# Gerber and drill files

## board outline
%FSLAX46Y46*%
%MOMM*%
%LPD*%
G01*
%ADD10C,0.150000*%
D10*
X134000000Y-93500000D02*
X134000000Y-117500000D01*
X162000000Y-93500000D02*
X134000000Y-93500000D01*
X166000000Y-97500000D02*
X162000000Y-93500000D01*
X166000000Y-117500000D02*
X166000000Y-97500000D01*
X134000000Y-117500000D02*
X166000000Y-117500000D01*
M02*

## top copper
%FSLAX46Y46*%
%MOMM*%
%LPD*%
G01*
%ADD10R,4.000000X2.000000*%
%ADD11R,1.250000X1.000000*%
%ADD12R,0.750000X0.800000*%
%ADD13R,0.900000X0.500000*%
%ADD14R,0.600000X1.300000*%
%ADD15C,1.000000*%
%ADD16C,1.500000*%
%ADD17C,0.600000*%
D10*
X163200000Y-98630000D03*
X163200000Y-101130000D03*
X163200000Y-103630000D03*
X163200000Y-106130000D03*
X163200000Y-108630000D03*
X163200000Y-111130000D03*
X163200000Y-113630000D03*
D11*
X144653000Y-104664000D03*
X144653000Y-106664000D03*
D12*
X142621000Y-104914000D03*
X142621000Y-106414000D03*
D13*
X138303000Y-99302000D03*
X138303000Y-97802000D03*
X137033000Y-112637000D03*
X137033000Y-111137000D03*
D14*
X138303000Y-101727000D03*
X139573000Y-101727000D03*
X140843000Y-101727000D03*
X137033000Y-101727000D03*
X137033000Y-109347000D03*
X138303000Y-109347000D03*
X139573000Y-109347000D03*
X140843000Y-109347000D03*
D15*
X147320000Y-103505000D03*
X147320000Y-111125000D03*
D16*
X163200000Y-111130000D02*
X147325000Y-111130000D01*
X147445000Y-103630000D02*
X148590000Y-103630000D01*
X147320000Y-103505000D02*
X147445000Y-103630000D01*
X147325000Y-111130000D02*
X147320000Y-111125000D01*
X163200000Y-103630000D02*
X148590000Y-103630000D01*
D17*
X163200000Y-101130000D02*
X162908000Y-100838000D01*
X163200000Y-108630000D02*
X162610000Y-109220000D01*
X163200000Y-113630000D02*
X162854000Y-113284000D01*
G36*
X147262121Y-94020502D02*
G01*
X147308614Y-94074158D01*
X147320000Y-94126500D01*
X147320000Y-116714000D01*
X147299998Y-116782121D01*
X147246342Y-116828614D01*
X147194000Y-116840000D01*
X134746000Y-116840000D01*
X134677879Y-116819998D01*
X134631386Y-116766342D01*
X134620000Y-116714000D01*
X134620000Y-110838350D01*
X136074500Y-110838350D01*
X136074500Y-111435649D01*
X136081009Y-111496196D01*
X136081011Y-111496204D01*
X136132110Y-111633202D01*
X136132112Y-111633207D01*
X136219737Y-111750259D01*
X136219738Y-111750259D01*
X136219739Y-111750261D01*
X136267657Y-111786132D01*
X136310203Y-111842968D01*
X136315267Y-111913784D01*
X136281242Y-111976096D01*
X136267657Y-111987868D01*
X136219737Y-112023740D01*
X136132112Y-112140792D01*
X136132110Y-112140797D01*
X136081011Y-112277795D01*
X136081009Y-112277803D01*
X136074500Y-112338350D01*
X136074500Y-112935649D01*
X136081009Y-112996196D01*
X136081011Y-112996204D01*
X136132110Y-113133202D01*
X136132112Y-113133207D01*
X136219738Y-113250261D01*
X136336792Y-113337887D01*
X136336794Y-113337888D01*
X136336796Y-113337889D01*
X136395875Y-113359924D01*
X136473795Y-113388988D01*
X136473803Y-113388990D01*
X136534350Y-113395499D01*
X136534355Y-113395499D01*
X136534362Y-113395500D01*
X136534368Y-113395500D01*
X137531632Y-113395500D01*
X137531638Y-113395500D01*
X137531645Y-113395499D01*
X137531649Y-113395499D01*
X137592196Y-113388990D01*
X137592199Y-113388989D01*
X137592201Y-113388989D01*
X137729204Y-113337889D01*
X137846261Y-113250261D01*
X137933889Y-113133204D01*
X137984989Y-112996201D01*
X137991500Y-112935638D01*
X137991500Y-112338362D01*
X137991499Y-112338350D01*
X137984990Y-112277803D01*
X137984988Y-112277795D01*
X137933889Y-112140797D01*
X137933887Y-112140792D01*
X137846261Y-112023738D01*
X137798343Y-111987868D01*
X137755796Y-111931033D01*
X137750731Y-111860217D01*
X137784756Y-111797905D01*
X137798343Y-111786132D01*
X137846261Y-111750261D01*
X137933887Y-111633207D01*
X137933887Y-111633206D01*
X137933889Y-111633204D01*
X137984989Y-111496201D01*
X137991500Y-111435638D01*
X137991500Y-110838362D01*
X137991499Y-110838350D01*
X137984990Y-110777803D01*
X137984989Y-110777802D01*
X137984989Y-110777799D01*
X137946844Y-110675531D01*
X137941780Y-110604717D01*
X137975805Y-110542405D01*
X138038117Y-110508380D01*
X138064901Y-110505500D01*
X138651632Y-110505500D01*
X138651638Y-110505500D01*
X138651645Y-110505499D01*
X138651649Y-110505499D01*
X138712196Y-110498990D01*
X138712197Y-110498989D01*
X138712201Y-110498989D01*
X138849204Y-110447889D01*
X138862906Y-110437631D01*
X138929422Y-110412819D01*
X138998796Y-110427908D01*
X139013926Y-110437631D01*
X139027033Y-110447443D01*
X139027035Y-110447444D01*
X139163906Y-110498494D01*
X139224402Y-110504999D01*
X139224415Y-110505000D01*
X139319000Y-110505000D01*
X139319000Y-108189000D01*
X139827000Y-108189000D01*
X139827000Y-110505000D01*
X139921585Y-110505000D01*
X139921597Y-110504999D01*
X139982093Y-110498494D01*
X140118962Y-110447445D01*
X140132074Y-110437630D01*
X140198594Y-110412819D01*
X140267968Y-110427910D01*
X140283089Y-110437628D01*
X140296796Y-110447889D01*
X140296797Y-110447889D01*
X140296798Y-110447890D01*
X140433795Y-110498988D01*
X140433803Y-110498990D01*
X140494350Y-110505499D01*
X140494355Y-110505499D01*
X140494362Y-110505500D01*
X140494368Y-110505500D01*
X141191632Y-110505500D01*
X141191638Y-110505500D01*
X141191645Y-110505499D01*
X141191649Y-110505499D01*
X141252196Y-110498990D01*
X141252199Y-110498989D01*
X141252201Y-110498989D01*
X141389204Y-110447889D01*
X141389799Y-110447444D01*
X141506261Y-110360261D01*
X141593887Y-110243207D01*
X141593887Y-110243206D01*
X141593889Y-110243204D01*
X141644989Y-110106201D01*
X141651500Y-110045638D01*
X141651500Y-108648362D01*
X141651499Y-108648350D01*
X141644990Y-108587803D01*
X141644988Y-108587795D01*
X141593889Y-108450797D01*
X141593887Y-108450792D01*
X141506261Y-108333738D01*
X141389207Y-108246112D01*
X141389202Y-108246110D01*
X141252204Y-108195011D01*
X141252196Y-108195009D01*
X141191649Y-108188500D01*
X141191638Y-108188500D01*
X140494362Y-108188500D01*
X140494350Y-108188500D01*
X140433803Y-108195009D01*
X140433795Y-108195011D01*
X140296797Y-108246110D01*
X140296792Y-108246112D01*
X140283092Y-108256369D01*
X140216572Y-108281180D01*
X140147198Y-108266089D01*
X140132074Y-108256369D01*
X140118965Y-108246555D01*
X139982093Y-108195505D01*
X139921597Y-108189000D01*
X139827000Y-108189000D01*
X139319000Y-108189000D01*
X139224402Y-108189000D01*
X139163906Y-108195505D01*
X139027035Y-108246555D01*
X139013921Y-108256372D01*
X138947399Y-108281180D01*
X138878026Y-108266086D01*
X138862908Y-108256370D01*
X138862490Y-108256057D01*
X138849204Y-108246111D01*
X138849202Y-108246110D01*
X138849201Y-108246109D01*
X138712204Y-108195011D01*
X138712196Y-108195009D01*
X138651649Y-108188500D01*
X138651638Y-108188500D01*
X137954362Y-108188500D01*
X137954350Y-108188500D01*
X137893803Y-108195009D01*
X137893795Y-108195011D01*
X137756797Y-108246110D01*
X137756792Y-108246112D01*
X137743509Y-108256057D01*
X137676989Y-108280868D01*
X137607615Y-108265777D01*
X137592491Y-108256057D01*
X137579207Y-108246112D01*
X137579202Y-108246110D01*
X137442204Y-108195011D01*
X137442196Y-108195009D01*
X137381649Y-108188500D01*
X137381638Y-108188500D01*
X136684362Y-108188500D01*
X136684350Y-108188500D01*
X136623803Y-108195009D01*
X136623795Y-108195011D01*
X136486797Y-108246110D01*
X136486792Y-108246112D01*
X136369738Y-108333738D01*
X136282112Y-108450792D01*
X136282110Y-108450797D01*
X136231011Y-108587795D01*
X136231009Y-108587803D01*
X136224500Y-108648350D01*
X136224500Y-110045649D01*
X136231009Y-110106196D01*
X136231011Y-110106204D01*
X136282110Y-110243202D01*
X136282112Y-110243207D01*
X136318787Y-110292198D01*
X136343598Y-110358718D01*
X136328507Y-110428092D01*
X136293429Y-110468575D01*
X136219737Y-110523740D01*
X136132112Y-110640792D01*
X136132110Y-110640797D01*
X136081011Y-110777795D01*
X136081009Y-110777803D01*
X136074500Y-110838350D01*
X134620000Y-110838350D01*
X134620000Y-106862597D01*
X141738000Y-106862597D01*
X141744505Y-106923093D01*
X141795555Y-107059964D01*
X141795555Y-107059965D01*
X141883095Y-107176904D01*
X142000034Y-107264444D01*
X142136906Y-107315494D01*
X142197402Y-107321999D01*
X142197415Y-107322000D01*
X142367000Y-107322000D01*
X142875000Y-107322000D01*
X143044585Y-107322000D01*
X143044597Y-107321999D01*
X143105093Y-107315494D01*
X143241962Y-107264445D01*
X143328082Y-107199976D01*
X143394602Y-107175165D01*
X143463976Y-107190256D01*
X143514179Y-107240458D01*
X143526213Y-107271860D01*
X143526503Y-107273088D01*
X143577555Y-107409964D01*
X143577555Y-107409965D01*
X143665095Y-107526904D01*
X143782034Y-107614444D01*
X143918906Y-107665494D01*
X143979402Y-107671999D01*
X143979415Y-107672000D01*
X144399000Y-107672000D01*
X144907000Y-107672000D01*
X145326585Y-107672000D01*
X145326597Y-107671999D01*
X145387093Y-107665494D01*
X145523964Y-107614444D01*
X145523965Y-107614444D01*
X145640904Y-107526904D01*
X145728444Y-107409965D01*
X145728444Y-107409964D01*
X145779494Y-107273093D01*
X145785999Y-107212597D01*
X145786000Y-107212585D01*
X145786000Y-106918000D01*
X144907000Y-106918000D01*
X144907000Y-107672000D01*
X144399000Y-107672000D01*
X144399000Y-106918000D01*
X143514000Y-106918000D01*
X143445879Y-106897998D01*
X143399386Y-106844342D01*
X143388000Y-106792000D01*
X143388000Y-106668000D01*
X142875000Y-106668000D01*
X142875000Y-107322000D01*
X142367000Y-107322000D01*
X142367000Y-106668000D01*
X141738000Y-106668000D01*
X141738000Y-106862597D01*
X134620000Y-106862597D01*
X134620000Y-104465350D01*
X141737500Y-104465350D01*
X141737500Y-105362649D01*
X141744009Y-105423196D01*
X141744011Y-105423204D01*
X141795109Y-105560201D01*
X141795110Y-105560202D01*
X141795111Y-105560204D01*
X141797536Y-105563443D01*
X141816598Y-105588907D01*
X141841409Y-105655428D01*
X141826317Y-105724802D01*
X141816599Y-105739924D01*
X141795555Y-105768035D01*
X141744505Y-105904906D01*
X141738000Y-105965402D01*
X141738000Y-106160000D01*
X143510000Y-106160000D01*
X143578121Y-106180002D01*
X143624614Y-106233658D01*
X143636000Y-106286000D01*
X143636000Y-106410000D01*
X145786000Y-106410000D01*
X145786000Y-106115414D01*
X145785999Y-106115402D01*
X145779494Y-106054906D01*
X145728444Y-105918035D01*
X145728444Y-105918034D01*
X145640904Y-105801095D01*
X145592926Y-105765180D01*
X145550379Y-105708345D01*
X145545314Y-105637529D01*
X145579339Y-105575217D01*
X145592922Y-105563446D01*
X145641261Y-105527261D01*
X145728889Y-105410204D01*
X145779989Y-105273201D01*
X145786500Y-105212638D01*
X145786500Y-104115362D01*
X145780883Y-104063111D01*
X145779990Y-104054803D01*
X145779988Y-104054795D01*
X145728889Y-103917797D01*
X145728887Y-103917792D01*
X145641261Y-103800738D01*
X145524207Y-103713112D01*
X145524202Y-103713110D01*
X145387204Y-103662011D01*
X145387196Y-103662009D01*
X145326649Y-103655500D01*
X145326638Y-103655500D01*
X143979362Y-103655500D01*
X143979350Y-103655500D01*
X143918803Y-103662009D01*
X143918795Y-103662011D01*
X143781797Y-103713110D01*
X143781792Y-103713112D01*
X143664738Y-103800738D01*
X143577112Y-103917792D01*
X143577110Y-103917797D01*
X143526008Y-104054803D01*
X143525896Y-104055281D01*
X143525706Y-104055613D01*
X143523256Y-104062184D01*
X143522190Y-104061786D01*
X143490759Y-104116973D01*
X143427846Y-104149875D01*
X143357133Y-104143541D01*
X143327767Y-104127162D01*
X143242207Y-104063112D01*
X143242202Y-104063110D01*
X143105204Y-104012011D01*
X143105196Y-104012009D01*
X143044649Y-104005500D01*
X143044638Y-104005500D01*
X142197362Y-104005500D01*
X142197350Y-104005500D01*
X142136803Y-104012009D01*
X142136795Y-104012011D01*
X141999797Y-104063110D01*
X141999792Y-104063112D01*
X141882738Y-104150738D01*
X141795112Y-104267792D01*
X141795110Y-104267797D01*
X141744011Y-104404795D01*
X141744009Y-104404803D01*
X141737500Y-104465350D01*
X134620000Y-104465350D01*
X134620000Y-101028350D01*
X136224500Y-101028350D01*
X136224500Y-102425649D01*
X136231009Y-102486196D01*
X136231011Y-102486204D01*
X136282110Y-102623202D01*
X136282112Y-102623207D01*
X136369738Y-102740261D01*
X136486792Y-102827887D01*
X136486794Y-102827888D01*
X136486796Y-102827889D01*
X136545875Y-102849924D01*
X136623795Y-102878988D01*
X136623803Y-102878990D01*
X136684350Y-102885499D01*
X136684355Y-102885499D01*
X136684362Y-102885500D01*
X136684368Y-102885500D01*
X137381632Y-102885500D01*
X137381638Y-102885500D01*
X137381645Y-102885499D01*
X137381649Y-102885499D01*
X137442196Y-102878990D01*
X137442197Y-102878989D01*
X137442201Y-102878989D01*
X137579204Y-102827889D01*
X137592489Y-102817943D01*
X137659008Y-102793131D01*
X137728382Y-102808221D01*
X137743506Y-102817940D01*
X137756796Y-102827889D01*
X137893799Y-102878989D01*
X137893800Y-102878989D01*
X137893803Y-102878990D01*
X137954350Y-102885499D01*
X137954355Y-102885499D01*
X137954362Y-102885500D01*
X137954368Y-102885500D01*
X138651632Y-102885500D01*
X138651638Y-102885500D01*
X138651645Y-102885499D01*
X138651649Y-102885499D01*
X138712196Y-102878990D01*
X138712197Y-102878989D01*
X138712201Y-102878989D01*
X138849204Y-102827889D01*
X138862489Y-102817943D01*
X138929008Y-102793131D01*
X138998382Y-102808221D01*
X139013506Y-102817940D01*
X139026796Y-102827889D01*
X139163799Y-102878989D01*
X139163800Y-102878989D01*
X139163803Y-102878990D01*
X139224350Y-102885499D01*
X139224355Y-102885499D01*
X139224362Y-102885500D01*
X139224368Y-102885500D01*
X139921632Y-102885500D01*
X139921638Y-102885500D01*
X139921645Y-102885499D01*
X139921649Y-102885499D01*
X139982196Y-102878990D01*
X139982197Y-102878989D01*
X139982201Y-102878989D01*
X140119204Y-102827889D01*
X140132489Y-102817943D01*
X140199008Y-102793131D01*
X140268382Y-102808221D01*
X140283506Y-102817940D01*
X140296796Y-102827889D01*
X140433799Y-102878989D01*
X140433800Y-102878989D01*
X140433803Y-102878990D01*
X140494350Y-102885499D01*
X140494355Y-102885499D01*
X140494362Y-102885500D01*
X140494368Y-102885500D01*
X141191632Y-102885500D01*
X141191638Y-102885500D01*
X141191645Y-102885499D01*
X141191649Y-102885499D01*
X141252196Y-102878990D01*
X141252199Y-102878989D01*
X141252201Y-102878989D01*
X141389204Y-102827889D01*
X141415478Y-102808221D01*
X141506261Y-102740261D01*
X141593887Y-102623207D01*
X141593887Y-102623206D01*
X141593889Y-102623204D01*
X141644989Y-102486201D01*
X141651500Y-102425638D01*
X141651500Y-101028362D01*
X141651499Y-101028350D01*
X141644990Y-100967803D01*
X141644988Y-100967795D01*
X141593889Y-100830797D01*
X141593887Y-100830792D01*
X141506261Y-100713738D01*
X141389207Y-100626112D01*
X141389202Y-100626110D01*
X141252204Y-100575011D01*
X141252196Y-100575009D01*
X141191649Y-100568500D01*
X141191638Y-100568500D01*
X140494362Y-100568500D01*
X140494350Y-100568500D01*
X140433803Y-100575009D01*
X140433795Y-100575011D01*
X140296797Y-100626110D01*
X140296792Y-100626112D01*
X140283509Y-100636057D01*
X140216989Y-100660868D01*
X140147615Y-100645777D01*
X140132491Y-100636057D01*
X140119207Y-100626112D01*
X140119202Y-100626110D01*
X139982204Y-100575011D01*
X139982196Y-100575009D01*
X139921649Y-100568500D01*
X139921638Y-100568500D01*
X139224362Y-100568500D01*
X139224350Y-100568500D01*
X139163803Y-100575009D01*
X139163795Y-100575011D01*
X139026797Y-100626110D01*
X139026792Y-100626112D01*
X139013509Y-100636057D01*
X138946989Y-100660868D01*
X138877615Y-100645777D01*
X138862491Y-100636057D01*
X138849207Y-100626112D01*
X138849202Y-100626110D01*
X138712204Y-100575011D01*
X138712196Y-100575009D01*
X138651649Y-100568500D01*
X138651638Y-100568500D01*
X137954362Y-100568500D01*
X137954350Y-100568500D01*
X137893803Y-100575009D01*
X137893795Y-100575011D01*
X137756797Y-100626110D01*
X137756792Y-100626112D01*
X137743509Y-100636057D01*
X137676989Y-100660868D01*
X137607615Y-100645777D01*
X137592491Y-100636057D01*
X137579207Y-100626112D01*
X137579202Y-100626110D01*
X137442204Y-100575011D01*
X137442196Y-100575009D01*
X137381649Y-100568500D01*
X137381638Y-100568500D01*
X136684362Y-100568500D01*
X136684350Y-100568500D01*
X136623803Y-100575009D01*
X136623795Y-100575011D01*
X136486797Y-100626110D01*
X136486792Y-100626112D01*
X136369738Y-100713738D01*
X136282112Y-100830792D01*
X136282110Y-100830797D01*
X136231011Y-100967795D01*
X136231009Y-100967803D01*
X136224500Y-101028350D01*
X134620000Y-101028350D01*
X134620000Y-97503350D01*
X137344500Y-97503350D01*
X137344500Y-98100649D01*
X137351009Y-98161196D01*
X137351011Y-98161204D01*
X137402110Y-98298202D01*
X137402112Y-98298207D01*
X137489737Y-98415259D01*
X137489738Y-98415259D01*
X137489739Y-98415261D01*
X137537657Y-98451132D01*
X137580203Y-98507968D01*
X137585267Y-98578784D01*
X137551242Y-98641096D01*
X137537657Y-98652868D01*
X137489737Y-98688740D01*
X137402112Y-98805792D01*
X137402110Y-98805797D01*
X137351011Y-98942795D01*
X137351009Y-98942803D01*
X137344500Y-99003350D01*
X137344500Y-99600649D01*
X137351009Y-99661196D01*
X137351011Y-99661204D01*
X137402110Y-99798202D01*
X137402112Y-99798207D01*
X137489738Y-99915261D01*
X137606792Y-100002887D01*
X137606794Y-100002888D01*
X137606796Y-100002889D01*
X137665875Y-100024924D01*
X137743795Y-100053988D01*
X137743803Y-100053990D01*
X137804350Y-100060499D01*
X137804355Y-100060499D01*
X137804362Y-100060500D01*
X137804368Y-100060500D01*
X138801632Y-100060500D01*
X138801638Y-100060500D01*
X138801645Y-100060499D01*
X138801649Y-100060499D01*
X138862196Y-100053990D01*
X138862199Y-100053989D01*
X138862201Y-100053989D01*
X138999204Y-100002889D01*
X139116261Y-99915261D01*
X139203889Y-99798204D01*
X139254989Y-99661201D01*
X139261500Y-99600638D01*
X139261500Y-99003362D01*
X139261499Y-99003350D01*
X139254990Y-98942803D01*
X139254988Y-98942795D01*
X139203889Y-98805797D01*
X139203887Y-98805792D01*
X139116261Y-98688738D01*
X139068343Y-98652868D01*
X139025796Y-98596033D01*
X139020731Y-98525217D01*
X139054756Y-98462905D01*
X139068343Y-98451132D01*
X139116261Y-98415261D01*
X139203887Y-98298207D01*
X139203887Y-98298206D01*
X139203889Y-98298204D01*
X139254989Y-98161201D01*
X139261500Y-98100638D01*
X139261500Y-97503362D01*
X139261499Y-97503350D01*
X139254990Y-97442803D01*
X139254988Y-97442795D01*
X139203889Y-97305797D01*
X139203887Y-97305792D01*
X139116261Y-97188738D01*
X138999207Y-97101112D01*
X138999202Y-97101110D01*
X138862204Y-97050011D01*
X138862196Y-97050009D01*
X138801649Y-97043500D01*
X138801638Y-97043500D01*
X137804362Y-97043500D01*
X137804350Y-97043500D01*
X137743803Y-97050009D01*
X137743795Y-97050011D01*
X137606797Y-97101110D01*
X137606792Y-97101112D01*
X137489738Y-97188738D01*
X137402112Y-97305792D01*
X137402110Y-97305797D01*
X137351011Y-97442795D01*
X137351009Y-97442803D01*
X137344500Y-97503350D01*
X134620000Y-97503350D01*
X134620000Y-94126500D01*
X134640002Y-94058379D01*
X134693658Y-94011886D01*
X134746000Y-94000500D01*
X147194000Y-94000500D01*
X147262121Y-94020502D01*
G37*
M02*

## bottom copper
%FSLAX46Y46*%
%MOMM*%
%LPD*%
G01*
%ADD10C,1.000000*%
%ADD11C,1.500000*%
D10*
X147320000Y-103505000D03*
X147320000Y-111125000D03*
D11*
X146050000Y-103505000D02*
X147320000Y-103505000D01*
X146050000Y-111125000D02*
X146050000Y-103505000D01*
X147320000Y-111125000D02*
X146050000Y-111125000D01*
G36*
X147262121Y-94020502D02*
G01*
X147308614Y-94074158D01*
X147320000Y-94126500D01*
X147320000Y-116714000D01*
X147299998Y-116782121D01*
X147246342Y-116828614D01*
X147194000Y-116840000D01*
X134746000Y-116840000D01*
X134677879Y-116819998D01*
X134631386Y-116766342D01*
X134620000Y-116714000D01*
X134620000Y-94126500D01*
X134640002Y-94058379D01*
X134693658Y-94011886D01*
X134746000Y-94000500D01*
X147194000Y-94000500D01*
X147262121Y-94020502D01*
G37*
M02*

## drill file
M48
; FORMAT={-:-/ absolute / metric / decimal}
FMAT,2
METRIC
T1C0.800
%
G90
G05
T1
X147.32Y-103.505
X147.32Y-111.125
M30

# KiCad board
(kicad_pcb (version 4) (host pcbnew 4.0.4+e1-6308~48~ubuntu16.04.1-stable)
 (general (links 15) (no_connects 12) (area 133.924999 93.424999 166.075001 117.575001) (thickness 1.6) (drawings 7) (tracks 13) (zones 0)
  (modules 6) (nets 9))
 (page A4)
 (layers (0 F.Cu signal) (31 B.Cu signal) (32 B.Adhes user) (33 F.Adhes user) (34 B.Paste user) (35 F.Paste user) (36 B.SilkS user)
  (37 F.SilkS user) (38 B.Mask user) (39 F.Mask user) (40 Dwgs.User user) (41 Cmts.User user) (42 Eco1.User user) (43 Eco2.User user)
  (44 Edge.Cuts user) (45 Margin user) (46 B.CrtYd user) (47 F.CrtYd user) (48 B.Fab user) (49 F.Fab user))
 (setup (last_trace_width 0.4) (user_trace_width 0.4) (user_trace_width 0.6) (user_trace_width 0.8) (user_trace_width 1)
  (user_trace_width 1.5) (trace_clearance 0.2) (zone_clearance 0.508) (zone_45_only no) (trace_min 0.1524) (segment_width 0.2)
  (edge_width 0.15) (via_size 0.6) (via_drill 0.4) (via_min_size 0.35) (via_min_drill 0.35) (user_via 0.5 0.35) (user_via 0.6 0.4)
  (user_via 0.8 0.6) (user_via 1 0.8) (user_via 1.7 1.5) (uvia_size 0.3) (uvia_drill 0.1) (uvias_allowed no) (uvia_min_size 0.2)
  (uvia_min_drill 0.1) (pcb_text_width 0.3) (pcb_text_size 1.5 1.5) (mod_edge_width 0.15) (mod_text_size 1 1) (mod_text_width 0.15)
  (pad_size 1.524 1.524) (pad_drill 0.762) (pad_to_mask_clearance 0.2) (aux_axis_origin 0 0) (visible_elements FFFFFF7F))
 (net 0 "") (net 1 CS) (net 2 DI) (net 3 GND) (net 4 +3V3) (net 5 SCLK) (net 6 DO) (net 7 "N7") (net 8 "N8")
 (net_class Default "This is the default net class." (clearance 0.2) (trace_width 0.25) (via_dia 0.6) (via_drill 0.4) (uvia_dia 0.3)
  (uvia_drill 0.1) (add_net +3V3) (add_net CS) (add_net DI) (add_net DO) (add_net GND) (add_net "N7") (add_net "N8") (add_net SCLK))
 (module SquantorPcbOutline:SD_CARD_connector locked (layer F.Cu) (at 163.2 106.13)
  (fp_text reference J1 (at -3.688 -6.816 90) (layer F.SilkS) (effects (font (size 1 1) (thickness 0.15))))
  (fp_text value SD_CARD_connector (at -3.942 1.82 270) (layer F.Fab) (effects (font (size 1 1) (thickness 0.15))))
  (pad 1 smd rect (at 0 -7.5 90) (size 2 4) (layers F.Cu F.Paste F.Mask) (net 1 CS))
  (pad 2 smd rect (at 0 -5 90) (size 2 4) (layers F.Cu F.Paste F.Mask) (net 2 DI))
  (pad 3 smd rect (at 0 -2.5 90) (size 2 4) (layers F.Cu F.Paste F.Mask) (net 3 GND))
  (pad 4 smd rect (at 0 0 90) (size 2 4) (layers F.Cu F.Paste F.Mask) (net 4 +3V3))
  (pad 5 smd rect (at 0 2.5 90) (size 2 4) (layers F.Cu F.Paste F.Mask) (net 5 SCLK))
  (pad 6 smd rect (at 0 5 90) (size 2 4) (layers F.Cu F.Paste F.Mask) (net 3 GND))
  (pad 7 smd rect (at 0 7.5 90) (size 2 4) (layers F.Cu F.Paste F.Mask) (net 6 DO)))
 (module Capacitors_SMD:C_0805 (layer F.Cu) (at 144.653 105.664 270)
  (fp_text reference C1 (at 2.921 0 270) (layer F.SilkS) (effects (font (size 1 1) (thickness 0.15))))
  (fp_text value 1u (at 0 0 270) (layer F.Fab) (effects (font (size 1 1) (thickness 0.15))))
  (pad 1 smd rect (at -1 0 270) (size 1 1.25) (layers F.Cu F.Paste F.Mask) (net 4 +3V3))
  (pad 2 smd rect (at 1 0 270) (size 1 1.25) (layers F.Cu F.Paste F.Mask) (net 3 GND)))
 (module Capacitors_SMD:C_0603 (layer F.Cu) (at 142.621 105.664 270)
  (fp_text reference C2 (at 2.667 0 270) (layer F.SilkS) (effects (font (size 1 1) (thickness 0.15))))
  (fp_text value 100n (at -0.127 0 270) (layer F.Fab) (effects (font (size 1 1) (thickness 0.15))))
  (pad 1 smd rect (at -0.75 0 270) (size 0.8 0.75) (layers F.Cu F.Paste F.Mask) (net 4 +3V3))
  (pad 2 smd rect (at 0.75 0 270) (size 0.8 0.75) (layers F.Cu F.Paste F.Mask) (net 3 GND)))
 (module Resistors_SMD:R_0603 (layer F.Cu) (at 138.303 98.552 90)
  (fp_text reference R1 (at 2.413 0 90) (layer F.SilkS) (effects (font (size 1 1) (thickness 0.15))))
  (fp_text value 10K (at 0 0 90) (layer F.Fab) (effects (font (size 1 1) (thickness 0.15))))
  (pad 1 smd rect (at -0.75 0 90) (size 0.5 0.9) (layers F.Cu F.Paste F.Mask) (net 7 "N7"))
  (pad 2 smd rect (at 0.75 0 90) (size 0.5 0.9) (layers F.Cu F.Paste F.Mask) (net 4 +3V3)))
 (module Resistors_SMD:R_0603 (layer F.Cu) (at 137.033 111.887 90)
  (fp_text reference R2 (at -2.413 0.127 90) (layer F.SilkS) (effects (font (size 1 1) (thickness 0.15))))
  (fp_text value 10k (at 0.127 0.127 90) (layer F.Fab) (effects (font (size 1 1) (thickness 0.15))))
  (pad 1 smd rect (at -0.75 0 90) (size 0.5 0.9) (layers F.Cu F.Paste F.Mask) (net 4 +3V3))
  (pad 2 smd rect (at 0.75 0 90) (size 0.5 0.9) (layers F.Cu F.Paste F.Mask) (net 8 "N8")))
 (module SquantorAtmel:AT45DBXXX (layer F.Cu) (at 138.938 105.537 270)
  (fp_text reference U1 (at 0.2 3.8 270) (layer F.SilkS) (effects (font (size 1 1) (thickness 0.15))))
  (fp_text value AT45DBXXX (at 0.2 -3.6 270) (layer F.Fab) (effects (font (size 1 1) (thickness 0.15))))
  (pad 3 smd rect (at -3.81 0.635 270) (size 1.3 0.6) (layers F.Cu F.Paste F.Mask) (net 7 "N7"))
  (pad 2 smd rect (at -3.81 -0.635 270) (size 1.3 0.6) (layers F.Cu F.Paste F.Mask) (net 5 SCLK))
  (pad 1 smd rect (at -3.81 -1.905 270) (size 1.3 0.6) (layers F.Cu F.Paste F.Mask) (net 2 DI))
  (pad 4 smd rect (at -3.81 1.905 270) (size 1.3 0.6) (layers F.Cu F.Paste F.Mask) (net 1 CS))
  (pad 5 smd rect (at 3.81 1.905 270) (size 1.3 0.6) (layers F.Cu F.Paste F.Mask) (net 8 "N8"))
  (pad 6 smd rect (at 3.81 0.635 270) (size 1.3 0.6) (layers F.Cu F.Paste F.Mask) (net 4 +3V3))
  (pad 7 smd rect (at 3.81 -0.635 270) (size 1.3 0.6) (layers F.Cu F.Paste F.Mask) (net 3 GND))
  (pad 8 smd rect (at 3.81 -1.905 270) (size 1.3 0.6) (layers F.Cu F.Paste F.Mask) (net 6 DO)))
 (gr_line (start 134 93.5) (end 134 117.5) (angle 90) (layer Edge.Cuts) (width 0.15))
 (gr_line (start 162 93.5) (end 134 93.5) (angle 90) (layer Edge.Cuts) (width 0.15))
 (gr_line (start 166 97.5) (end 162 93.5) (angle 90) (layer Edge.Cuts) (width 0.15))
 (gr_line (start 166 117.5) (end 166 97.5) (angle 90) (layer Edge.Cuts) (width 0.15))
 (gr_line (start 134 117.5) (end 166 117.5) (angle 90) (layer Edge.Cuts) (width 0.15))
 (segment (start 163.2 111.13) (end 147.325 111.13) (width 1.5) (layer F.Cu) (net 3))
 (segment (start 147.445 103.63) (end 148.59 103.63) (width 1.5) (layer F.Cu) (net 3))
 (segment (start 147.32 103.505) (end 147.445 103.63) (width 1.5) (layer F.Cu) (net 3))
 (via (at 147.32 103.505) (size 1) (drill 0.8) (layers F.Cu B.Cu) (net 3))
 (segment (start 146.05 103.505) (end 147.32 103.505) (width 1.5) (layer B.Cu) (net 3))
 (segment (start 146.05 111.125) (end 146.05 103.505) (width 1.5) (layer B.Cu) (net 3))
 (segment (start 147.32 111.125) (end 146.05 111.125) (width 1.5) (layer B.Cu) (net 3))
 (via (at 147.32 111.125) (size 1) (drill 0.8) (layers F.Cu B.Cu) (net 3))
 (segment (start 147.325 111.13) (end 147.32 111.125) (width 1.5) (layer F.Cu) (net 3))
 (segment (start 163.2 103.63) (end 148.59 103.63) (width 1.5) (layer F.Cu) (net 3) (status 10))
 (segment (start 163.2 101.13) (end 162.908 100.838) (width 0.6) (layer F.Cu) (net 2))
 (segment (start 163.2 108.63) (end 162.61 109.22) (width 0.6) (layer F.Cu) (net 5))
 (segment (start 163.2 113.63) (end 162.854 113.284) (width 0.6) (layer F.Cu) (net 6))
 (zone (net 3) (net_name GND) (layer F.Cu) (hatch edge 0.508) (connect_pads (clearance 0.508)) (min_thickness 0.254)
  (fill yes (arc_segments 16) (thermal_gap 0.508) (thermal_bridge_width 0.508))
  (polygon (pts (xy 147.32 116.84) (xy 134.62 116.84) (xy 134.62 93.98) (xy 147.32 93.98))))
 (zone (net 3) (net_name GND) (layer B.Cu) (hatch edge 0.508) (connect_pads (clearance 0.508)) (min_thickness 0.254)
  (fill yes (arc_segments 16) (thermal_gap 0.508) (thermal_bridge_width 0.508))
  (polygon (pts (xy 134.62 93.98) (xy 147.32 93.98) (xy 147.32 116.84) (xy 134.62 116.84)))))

